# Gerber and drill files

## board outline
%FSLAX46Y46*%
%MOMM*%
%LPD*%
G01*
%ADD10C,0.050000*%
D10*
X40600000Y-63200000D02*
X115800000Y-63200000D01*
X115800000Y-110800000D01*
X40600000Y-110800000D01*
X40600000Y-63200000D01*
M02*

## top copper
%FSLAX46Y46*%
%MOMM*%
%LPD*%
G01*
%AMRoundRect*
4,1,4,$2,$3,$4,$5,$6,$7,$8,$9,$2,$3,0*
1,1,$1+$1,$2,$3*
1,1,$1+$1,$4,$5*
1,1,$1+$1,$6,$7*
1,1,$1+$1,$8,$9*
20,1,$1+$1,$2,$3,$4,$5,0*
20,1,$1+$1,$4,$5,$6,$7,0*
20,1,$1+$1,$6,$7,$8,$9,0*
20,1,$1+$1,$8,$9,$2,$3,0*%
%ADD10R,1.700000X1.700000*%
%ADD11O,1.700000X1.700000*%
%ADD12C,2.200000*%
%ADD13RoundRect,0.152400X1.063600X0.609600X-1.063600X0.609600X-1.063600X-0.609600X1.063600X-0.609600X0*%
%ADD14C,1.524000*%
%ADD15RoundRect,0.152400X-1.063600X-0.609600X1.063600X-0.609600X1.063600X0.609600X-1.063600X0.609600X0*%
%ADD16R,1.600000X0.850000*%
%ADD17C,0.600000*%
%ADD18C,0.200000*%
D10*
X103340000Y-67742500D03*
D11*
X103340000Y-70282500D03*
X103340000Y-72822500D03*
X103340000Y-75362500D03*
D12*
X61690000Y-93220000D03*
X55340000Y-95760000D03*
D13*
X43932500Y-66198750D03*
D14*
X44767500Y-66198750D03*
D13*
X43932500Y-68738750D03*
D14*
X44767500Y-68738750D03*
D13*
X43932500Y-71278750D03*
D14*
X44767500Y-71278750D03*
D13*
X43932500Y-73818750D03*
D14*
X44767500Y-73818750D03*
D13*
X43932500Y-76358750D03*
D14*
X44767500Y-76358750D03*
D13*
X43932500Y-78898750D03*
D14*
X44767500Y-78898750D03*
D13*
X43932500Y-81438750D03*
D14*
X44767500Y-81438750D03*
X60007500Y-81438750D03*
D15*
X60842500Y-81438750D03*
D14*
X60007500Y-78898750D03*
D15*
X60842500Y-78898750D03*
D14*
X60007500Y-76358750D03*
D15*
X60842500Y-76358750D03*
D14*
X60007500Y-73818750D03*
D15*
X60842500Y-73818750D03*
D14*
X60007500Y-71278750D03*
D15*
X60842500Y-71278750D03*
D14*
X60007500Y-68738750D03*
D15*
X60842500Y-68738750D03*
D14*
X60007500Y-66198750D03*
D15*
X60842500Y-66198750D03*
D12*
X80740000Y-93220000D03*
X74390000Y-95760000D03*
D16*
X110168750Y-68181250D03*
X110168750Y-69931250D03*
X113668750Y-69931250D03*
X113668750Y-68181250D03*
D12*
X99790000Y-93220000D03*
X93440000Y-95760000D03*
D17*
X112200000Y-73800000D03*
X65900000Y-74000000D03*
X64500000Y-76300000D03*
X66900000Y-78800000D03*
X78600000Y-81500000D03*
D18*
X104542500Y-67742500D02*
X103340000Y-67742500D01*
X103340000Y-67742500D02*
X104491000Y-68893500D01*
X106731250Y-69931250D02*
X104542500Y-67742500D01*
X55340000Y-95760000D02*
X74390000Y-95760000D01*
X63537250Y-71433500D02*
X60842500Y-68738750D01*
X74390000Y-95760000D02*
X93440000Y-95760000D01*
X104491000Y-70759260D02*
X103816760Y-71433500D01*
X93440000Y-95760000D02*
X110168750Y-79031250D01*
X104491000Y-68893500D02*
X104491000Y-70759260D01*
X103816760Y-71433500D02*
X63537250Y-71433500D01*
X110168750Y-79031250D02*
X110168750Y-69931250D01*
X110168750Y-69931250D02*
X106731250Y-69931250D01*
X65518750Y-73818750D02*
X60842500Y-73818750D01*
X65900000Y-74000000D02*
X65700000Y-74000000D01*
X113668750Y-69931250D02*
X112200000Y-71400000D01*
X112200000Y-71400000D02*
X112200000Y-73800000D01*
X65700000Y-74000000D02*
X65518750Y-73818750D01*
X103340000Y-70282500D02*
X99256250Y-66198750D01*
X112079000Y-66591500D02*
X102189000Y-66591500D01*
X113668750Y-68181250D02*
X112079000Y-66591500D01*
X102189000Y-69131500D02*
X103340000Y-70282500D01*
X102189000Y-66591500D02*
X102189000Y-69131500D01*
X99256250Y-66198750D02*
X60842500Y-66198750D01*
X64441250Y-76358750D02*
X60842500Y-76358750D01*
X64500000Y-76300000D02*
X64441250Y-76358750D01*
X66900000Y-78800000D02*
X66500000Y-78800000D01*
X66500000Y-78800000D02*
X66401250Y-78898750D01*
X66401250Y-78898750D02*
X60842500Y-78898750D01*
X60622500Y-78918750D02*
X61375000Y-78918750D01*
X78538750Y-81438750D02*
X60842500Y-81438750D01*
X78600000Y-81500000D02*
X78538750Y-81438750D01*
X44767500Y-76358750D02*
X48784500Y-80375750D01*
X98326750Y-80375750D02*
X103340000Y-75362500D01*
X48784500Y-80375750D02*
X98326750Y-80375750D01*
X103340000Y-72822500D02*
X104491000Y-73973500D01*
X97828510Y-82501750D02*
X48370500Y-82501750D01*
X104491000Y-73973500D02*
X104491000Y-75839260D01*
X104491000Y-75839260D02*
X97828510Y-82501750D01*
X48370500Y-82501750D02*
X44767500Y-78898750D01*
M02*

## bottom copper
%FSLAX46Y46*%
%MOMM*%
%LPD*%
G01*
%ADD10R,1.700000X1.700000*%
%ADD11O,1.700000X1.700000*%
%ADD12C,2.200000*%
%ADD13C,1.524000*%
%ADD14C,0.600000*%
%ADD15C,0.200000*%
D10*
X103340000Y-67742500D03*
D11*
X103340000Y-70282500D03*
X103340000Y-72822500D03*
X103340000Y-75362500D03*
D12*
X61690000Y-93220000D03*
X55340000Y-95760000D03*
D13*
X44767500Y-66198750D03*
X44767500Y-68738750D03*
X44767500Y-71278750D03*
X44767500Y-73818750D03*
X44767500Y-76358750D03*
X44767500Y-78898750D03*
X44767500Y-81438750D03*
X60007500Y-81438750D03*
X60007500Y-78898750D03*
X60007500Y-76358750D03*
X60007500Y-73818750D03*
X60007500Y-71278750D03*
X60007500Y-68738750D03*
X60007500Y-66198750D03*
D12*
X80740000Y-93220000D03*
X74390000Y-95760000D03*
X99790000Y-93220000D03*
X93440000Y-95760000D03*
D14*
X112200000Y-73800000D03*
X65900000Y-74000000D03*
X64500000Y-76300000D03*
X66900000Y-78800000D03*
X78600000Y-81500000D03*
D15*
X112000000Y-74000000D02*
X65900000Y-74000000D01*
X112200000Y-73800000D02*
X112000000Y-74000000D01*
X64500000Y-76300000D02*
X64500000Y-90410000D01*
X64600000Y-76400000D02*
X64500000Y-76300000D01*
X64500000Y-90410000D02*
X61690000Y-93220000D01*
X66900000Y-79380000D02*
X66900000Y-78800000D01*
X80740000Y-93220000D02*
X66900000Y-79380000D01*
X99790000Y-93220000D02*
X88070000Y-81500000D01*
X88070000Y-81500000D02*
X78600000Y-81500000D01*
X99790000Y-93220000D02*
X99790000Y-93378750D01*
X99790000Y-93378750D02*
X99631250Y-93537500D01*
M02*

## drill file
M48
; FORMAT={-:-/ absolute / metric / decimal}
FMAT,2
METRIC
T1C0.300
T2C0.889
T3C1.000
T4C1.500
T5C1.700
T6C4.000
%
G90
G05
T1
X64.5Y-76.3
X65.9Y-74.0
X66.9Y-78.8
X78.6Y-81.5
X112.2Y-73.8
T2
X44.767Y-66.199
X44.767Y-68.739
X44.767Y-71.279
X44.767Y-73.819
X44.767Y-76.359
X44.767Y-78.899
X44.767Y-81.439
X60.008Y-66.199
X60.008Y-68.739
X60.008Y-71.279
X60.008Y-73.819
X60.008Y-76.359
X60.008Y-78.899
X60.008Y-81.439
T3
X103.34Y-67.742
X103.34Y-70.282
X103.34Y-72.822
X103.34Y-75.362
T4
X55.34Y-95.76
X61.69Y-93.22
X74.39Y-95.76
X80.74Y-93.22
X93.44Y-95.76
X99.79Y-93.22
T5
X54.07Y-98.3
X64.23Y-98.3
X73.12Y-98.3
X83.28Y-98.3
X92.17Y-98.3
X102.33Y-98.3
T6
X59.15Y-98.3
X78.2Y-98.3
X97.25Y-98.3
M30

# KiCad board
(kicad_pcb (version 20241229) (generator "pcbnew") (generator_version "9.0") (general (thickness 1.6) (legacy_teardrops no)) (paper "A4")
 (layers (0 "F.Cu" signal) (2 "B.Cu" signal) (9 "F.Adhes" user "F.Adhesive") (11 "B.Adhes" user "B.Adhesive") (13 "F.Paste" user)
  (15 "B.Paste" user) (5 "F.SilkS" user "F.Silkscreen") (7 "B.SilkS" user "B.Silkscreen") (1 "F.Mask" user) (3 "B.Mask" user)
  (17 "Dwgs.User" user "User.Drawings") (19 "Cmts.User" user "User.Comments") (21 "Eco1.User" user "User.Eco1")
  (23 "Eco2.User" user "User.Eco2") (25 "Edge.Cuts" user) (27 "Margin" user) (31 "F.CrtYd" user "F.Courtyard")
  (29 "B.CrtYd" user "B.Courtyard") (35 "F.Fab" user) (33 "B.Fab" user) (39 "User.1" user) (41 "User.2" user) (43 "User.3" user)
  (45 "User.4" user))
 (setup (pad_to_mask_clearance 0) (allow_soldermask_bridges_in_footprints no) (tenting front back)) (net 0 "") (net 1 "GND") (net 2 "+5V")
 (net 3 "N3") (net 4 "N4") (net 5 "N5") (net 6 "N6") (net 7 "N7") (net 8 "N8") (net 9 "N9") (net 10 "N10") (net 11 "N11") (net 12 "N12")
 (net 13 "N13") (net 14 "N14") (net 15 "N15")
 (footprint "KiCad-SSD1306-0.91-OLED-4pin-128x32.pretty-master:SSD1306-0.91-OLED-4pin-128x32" (layer "F.Cu") (at 66.84 65.5525)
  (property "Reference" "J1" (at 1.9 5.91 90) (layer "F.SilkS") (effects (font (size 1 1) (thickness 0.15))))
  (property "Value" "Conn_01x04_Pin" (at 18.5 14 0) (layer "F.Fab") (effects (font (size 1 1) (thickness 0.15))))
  (pad "1" thru_hole rect (at 36.5 2.19) (size 1.7 1.7) (drill 1) (layers "*.Cu" "*.Mask") (remove_unused_layers no) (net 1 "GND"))
  (pad "2" thru_hole oval (at 36.5 4.73) (size 1.7 1.7) (drill 1) (layers "*.Cu" "*.Mask") (remove_unused_layers no) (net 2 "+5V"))
  (pad "3" thru_hole oval (at 36.5 7.27) (size 1.7 1.7) (drill 1) (layers "*.Cu" "*.Mask") (remove_unused_layers no) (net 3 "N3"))
  (pad "4" thru_hole oval (at 36.5 9.81) (size 1.7 1.7) (drill 1) (layers "*.Cu" "*.Mask") (remove_unused_layers no) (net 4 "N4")))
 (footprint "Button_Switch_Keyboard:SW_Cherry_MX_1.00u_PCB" (layer "F.Cu") (at 61.69 93.22)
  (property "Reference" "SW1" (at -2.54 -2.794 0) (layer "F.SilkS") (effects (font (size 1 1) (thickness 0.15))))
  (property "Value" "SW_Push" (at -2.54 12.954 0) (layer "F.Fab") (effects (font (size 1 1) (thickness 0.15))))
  (pad "" np_thru_hole circle (at -7.62 5.08) (size 1.7 1.7) (drill 1.7) (layers "*.Cu" "*.Mask"))
  (pad "" np_thru_hole circle (at -2.54 5.08) (size 4 4) (drill 4) (layers "*.Cu" "*.Mask"))
  (pad "" np_thru_hole circle (at 2.54 5.08) (size 1.7 1.7) (drill 1.7) (layers "*.Cu" "*.Mask"))
  (pad "1" thru_hole circle (at 0 0) (size 2.2 2.2) (drill 1.5) (layers "*.Cu" "*.Mask") (remove_unused_layers no) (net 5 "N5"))
  (pad "2" thru_hole circle (at -6.35 2.54) (size 2.2 2.2) (drill 1.5) (layers "*.Cu" "*.Mask") (remove_unused_layers no) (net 1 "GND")))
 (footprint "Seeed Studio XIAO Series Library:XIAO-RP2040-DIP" (layer "F.Cu") (at 52.3875 73.81875)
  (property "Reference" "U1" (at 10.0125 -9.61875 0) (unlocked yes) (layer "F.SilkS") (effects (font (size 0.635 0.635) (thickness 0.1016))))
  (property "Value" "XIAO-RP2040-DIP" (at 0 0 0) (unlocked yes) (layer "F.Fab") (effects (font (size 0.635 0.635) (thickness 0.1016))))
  (pad "1" smd roundrect (at -8.455 -7.62 180) (size 2.432 1.524) (layers "F.Cu" "F.Mask") (roundrect_rratio 0.1) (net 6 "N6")
   (thermal_bridge_angle 45))
  (pad "1" thru_hole circle (at -7.62 -7.62 180) (size 1.524 1.524) (drill 0.889) (layers "*.Cu" "*.Mask") (remove_unused_layers no)
   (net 6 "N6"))
  (pad "2" smd roundrect (at -8.455 -5.08 180) (size 2.432 1.524) (layers "F.Cu" "F.Mask") (roundrect_rratio 0.1) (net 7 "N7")
   (thermal_bridge_angle 45))
  (pad "2" thru_hole circle (at -7.62 -5.08 180) (size 1.524 1.524) (drill 0.889) (layers "*.Cu" "*.Mask") (remove_unused_layers no)
   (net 7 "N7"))
  (pad "3" smd roundrect (at -8.455 -2.54 180) (size 2.432 1.524) (layers "F.Cu" "F.Mask") (roundrect_rratio 0.1) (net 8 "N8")
   (thermal_bridge_angle 45))
  (pad "3" thru_hole circle (at -7.62 -2.54 180) (size 1.524 1.524) (drill 0.889) (layers "*.Cu" "*.Mask") (remove_unused_layers no)
   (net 8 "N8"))
  (pad "4" smd roundrect (at -8.455 0 180) (size 2.432 1.524) (layers "F.Cu" "F.Mask") (roundrect_rratio 0.1) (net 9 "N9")
   (thermal_bridge_angle 45))
  (pad "4" thru_hole circle (at -7.62 0 180) (size 1.524 1.524) (drill 0.889) (layers "*.Cu" "*.Mask") (remove_unused_layers no)
   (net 9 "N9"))
  (pad "5" smd roundrect (at -8.455 2.54 180) (size 2.432 1.524) (layers "F.Cu" "F.Mask") (roundrect_rratio 0.1) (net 4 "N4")
   (thermal_bridge_angle 45))
  (pad "5" thru_hole circle (at -7.62 2.54 180) (size 1.524 1.524) (drill 0.889) (layers "*.Cu" "*.Mask") (remove_unused_layers no)
   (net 4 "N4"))
  (pad "6" smd roundrect (at -8.455 5.08 180) (size 2.432 1.524) (layers "F.Cu" "F.Mask") (roundrect_rratio 0.1) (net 3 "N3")
   (thermal_bridge_angle 45))
  (pad "6" thru_hole circle (at -7.62 5.08 180) (size 1.524 1.524) (drill 0.889) (layers "*.Cu" "*.Mask") (remove_unused_layers no)
   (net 3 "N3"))
  (pad "7" smd roundrect (at -8.455 7.62 180) (size 2.432 1.524) (layers "F.Cu" "F.Mask") (roundrect_rratio 0.1) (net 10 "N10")
   (thermal_bridge_angle 45))
  (pad "7" thru_hole circle (at -7.62 7.62 180) (size 1.524 1.524) (drill 0.889) (layers "*.Cu" "*.Mask") (remove_unused_layers no)
   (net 10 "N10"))
  (pad "8" thru_hole circle (at 7.62 7.62) (size 1.524 1.524) (drill 0.889) (layers "*.Cu" "*.Mask") (remove_unused_layers no)
   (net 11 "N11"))
  (pad "8" smd roundrect (at 8.455 7.62) (size 2.432 1.524) (layers "F.Cu" "F.Mask") (roundrect_rratio 0.1) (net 11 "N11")
   (thermal_bridge_angle 45))
  (pad "9" thru_hole circle (at 7.62 5.08) (size 1.524 1.524) (drill 0.889) (layers "*.Cu" "*.Mask") (remove_unused_layers no)
   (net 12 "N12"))
  (pad "9" smd roundrect (at 8.455 5.08) (size 2.432 1.524) (layers "F.Cu" "F.Mask") (roundrect_rratio 0.1) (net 12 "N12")
   (thermal_bridge_angle 45))
  (pad "10" thru_hole circle (at 7.62 2.54) (size 1.524 1.524) (drill 0.889) (layers "*.Cu" "*.Mask") (remove_unused_layers no) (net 5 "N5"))
  (pad "10" smd roundrect (at 8.455 2.54) (size 2.432 1.524) (layers "F.Cu" "F.Mask") (roundrect_rratio 0.1) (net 5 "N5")
   (thermal_bridge_angle 45))
  (pad "11" thru_hole circle (at 7.62 0) (size 1.524 1.524) (drill 0.889) (layers "*.Cu" "*.Mask") (remove_unused_layers no) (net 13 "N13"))
  (pad "11" smd roundrect (at 8.455 0) (size 2.432 1.524) (layers "F.Cu" "F.Mask") (roundrect_rratio 0.1) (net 13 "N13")
   (thermal_bridge_angle 45))
  (pad "12" thru_hole circle (at 7.62 -2.54) (size 1.524 1.524) (drill 0.889) (layers "*.Cu" "*.Mask") (remove_unused_layers no)
   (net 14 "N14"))
  (pad "12" smd roundrect (at 8.455 -2.54) (size 2.432 1.524) (layers "F.Cu" "F.Mask") (roundrect_rratio 0.1) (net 14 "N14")
   (thermal_bridge_angle 45))
  (pad "13" thru_hole circle (at 7.62 -5.08) (size 1.524 1.524) (drill 0.889) (layers "*.Cu" "*.Mask") (remove_unused_layers no)
   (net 1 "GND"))
  (pad "13" smd roundrect (at 8.455 -5.08) (size 2.432 1.524) (layers "F.Cu" "F.Mask") (roundrect_rratio 0.1) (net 1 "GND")
   (thermal_bridge_angle 45))
  (pad "14" thru_hole circle (at 7.62 -7.62) (size 1.524 1.524) (drill 0.889) (layers "*.Cu" "*.Mask") (remove_unused_layers no)
   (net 2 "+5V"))
  (pad "14" smd roundrect (at 8.455 -7.62) (size 2.432 1.524) (layers "F.Cu" "F.Mask") (roundrect_rratio 0.1) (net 2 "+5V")
   (thermal_bridge_angle 45)))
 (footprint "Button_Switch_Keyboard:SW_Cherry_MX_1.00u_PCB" (layer "F.Cu") (at 80.74 93.22)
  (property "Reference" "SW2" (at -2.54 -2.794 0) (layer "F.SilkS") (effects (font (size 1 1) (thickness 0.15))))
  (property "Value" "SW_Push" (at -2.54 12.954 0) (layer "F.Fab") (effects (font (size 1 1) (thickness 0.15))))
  (pad "" np_thru_hole circle (at -7.62 5.08) (size 1.7 1.7) (drill 1.7) (layers "*.Cu" "*.Mask"))
  (pad "" np_thru_hole circle (at -2.54 5.08) (size 4 4) (drill 4) (layers "*.Cu" "*.Mask"))
  (pad "" np_thru_hole circle (at 2.54 5.08) (size 1.7 1.7) (drill 1.7) (layers "*.Cu" "*.Mask"))
  (pad "1" thru_hole circle (at 0 0) (size 2.2 2.2) (drill 1.5) (layers "*.Cu" "*.Mask") (remove_unused_layers no) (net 12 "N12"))
  (pad "2" thru_hole circle (at -6.35 2.54) (size 2.2 2.2) (drill 1.5) (layers "*.Cu" "*.Mask") (remove_unused_layers no) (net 1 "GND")))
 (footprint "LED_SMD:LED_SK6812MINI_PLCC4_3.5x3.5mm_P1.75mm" (layer "F.Cu") (at 111.91875 69.05625)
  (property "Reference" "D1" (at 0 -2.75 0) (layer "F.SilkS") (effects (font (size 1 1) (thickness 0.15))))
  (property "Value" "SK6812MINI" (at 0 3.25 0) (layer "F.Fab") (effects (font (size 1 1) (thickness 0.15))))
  (pad "1" smd rect (at -1.75 -0.875) (size 1.6 0.85) (layers "F.Cu" "F.Mask" "F.Paste") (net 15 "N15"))
  (pad "2" smd rect (at -1.75 0.875) (size 1.6 0.85) (layers "F.Cu" "F.Mask" "F.Paste") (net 1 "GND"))
  (pad "3" smd rect (at 1.75 0.875) (size 1.6 0.85) (layers "F.Cu" "F.Mask" "F.Paste") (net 13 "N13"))
  (pad "4" smd rect (at 1.75 -0.875) (size 1.6 0.85) (layers "F.Cu" "F.Mask" "F.Paste") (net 2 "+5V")))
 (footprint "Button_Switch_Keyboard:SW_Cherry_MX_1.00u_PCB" (layer "F.Cu") (at 99.79 93.22)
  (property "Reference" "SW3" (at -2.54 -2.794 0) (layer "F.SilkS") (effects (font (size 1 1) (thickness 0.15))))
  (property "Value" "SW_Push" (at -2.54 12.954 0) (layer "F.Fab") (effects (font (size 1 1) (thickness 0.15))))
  (pad "" np_thru_hole circle (at -7.62 5.08) (size 1.7 1.7) (drill 1.7) (layers "*.Cu" "*.Mask"))
  (pad "" np_thru_hole circle (at -2.54 5.08) (size 4 4) (drill 4) (layers "*.Cu" "*.Mask"))
  (pad "" np_thru_hole circle (at 2.54 5.08) (size 1.7 1.7) (drill 1.7) (layers "*.Cu" "*.Mask"))
  (pad "1" thru_hole circle (at 0 0) (size 2.2 2.2) (drill 1.5) (layers "*.Cu" "*.Mask") (remove_unused_layers no) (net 11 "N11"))
  (pad "2" thru_hole circle (at -6.35 2.54) (size 2.2 2.2) (drill 1.5) (layers "*.Cu" "*.Mask") (remove_unused_layers no) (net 1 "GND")))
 (gr_rect (start 40.6 63.2) (end 115.8 110.8) (stroke (width 0.05) (type default)) (fill no) (layer "Edge.Cuts"))
 (segment (start 104.5425 67.7425) (end 103.34 67.7425) (width 0.2) (layer "F.Cu") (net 1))
 (segment (start 103.34 67.7425) (end 104.491 68.8935) (width 0.2) (layer "F.Cu") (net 1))
 (segment (start 106.73125 69.93125) (end 104.5425 67.7425) (width 0.2) (layer "F.Cu") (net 1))
 (segment (start 55.34 95.76) (end 74.39 95.76) (width 0.2) (layer "F.Cu") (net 1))
 (segment (start 63.53725 71.4335) (end 60.8425 68.73875) (width 0.2) (layer "F.Cu") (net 1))
 (segment (start 74.39 95.76) (end 93.44 95.76) (width 0.2) (layer "F.Cu") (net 1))
 (segment (start 104.491 70.75926) (end 103.81676 71.4335) (width 0.2) (layer "F.Cu") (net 1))
 (segment (start 93.44 95.76) (end 110.16875 79.03125) (width 0.2) (layer "F.Cu") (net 1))
 (segment (start 104.491 68.8935) (end 104.491 70.75926) (width 0.2) (layer "F.Cu") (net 1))
 (segment (start 103.81676 71.4335) (end 63.53725 71.4335) (width 0.2) (layer "F.Cu") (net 1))
 (segment (start 110.16875 79.03125) (end 110.16875 69.93125) (width 0.2) (layer "F.Cu") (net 1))
 (segment (start 110.16875 69.93125) (end 106.73125 69.93125) (width 0.2) (layer "F.Cu") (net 1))
 (segment (start 65.51875 73.81875) (end 60.8425 73.81875) (width 0.2) (layer "F.Cu") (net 13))
 (segment (start 65.9 74) (end 65.7 74) (width 0.2) (layer "F.Cu") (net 13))
 (segment (start 113.66875 69.93125) (end 112.2 71.4) (width 0.2) (layer "F.Cu") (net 13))
 (segment (start 112.2 71.4) (end 112.2 73.8) (width 0.2) (layer "F.Cu") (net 13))
 (segment (start 65.7 74) (end 65.51875 73.81875) (width 0.2) (layer "F.Cu") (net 13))
 (via (at 112.2 73.8) (size 0.6) (drill 0.3) (layers "F.Cu" "B.Cu") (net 13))
 (via (at 65.9 74) (size 0.6) (drill 0.3) (layers "F.Cu" "B.Cu") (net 13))
 (segment (start 112 74) (end 65.9 74) (width 0.2) (layer "B.Cu") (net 13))
 (segment (start 112.2 73.8) (end 112 74) (width 0.2) (layer "B.Cu") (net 13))
 (segment (start 103.34 70.2825) (end 99.25625 66.19875) (width 0.2) (layer "F.Cu") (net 2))
 (segment (start 112.079 66.5915) (end 102.189 66.5915) (width 0.2) (layer "F.Cu") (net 2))
 (segment (start 113.66875 68.18125) (end 112.079 66.5915) (width 0.2) (layer "F.Cu") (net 2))
 (segment (start 102.189 69.1315) (end 103.34 70.2825) (width 0.2) (layer "F.Cu") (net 2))
 (segment (start 102.189 66.5915) (end 102.189 69.1315) (width 0.2) (layer "F.Cu") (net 2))
 (segment (start 99.25625 66.19875) (end 60.8425 66.19875) (width 0.2) (layer "F.Cu") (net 2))
 (segment (start 64.44125 76.35875) (end 60.8425 76.35875) (width 0.2) (layer "F.Cu") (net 5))
 (segment (start 64.5 76.3) (end 64.44125 76.35875) (width 0.2) (layer "F.Cu") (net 5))
 (via (at 64.5 76.3) (size 0.6) (drill 0.3) (layers "F.Cu" "B.Cu") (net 5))
 (segment (start 64.5 76.3) (end 64.5 90.41) (width 0.2) (layer "B.Cu") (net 5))
 (segment (start 64.6 76.4) (end 64.5 76.3) (width 0.2) (layer "B.Cu") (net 5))
 (segment (start 64.5 90.41) (end 61.69 93.22) (width 0.2) (layer "B.Cu") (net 5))
 (segment (start 66.9 78.8) (end 66.5 78.8) (width 0.2) (layer "F.Cu") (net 12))
 (segment (start 66.5 78.8) (end 66.40125 78.89875) (width 0.2) (layer "F.Cu") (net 12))
 (segment (start 66.40125 78.89875) (end 60.8425 78.89875) (width 0.2) (layer "F.Cu") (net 12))
 (segment (start 60.6225 78.91875) (end 61.375 78.91875) (width 0.2) (layer "F.Cu") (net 12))
 (via (at 66.9 78.8) (size 0.6) (drill 0.3) (layers "F.Cu" "B.Cu") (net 12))
 (segment (start 66.9 79.38) (end 66.9 78.8) (width 0.2) (layer "B.Cu") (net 12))
 (segment (start 80.74 93.22) (end 66.9 79.38) (width 0.2) (layer "B.Cu") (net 12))
 (segment (start 78.53875 81.43875) (end 60.8425 81.43875) (width 0.2) (layer "F.Cu") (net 11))
 (segment (start 78.6 81.5) (end 78.53875 81.43875) (width 0.2) (layer "F.Cu") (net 11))
 (via (at 78.6 81.5) (size 0.6) (drill 0.3) (layers "F.Cu" "B.Cu") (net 11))
 (segment (start 99.79 93.22) (end 88.07 81.5) (width 0.2) (layer "B.Cu") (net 11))
 (segment (start 88.07 81.5) (end 78.6 81.5) (width 0.2) (layer "B.Cu") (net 11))
 (segment (start 99.79 93.22) (end 99.79 93.37875) (width 0.2) (layer "B.Cu") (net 11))
 (segment (start 99.79 93.37875) (end 99.63125 93.5375) (width 0.2) (layer "B.Cu") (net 11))
 (segment (start 44.7675 76.35875) (end 48.7845 80.37575) (width 0.2) (layer "F.Cu") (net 4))
 (segment (start 98.32675 80.37575) (end 103.34 75.3625) (width 0.2) (layer "F.Cu") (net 4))
 (segment (start 48.7845 80.37575) (end 98.32675 80.37575) (width 0.2) (layer "F.Cu") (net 4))
 (segment (start 103.34 72.8225) (end 104.491 73.9735) (width 0.2) (layer "F.Cu") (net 3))
 (segment (start 97.82851 82.50175) (end 48.3705 82.50175) (width 0.2) (layer "F.Cu") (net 3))
 (segment (start 104.491 73.9735) (end 104.491 75.83926) (width 0.2) (layer "F.Cu") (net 3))
 (segment (start 104.491 75.83926) (end 97.82851 82.50175) (width 0.2) (layer "F.Cu") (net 3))
 (segment (start 48.3705 82.50175) (end 44.7675 78.89875) (width 0.2) (layer "F.Cu") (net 3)))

